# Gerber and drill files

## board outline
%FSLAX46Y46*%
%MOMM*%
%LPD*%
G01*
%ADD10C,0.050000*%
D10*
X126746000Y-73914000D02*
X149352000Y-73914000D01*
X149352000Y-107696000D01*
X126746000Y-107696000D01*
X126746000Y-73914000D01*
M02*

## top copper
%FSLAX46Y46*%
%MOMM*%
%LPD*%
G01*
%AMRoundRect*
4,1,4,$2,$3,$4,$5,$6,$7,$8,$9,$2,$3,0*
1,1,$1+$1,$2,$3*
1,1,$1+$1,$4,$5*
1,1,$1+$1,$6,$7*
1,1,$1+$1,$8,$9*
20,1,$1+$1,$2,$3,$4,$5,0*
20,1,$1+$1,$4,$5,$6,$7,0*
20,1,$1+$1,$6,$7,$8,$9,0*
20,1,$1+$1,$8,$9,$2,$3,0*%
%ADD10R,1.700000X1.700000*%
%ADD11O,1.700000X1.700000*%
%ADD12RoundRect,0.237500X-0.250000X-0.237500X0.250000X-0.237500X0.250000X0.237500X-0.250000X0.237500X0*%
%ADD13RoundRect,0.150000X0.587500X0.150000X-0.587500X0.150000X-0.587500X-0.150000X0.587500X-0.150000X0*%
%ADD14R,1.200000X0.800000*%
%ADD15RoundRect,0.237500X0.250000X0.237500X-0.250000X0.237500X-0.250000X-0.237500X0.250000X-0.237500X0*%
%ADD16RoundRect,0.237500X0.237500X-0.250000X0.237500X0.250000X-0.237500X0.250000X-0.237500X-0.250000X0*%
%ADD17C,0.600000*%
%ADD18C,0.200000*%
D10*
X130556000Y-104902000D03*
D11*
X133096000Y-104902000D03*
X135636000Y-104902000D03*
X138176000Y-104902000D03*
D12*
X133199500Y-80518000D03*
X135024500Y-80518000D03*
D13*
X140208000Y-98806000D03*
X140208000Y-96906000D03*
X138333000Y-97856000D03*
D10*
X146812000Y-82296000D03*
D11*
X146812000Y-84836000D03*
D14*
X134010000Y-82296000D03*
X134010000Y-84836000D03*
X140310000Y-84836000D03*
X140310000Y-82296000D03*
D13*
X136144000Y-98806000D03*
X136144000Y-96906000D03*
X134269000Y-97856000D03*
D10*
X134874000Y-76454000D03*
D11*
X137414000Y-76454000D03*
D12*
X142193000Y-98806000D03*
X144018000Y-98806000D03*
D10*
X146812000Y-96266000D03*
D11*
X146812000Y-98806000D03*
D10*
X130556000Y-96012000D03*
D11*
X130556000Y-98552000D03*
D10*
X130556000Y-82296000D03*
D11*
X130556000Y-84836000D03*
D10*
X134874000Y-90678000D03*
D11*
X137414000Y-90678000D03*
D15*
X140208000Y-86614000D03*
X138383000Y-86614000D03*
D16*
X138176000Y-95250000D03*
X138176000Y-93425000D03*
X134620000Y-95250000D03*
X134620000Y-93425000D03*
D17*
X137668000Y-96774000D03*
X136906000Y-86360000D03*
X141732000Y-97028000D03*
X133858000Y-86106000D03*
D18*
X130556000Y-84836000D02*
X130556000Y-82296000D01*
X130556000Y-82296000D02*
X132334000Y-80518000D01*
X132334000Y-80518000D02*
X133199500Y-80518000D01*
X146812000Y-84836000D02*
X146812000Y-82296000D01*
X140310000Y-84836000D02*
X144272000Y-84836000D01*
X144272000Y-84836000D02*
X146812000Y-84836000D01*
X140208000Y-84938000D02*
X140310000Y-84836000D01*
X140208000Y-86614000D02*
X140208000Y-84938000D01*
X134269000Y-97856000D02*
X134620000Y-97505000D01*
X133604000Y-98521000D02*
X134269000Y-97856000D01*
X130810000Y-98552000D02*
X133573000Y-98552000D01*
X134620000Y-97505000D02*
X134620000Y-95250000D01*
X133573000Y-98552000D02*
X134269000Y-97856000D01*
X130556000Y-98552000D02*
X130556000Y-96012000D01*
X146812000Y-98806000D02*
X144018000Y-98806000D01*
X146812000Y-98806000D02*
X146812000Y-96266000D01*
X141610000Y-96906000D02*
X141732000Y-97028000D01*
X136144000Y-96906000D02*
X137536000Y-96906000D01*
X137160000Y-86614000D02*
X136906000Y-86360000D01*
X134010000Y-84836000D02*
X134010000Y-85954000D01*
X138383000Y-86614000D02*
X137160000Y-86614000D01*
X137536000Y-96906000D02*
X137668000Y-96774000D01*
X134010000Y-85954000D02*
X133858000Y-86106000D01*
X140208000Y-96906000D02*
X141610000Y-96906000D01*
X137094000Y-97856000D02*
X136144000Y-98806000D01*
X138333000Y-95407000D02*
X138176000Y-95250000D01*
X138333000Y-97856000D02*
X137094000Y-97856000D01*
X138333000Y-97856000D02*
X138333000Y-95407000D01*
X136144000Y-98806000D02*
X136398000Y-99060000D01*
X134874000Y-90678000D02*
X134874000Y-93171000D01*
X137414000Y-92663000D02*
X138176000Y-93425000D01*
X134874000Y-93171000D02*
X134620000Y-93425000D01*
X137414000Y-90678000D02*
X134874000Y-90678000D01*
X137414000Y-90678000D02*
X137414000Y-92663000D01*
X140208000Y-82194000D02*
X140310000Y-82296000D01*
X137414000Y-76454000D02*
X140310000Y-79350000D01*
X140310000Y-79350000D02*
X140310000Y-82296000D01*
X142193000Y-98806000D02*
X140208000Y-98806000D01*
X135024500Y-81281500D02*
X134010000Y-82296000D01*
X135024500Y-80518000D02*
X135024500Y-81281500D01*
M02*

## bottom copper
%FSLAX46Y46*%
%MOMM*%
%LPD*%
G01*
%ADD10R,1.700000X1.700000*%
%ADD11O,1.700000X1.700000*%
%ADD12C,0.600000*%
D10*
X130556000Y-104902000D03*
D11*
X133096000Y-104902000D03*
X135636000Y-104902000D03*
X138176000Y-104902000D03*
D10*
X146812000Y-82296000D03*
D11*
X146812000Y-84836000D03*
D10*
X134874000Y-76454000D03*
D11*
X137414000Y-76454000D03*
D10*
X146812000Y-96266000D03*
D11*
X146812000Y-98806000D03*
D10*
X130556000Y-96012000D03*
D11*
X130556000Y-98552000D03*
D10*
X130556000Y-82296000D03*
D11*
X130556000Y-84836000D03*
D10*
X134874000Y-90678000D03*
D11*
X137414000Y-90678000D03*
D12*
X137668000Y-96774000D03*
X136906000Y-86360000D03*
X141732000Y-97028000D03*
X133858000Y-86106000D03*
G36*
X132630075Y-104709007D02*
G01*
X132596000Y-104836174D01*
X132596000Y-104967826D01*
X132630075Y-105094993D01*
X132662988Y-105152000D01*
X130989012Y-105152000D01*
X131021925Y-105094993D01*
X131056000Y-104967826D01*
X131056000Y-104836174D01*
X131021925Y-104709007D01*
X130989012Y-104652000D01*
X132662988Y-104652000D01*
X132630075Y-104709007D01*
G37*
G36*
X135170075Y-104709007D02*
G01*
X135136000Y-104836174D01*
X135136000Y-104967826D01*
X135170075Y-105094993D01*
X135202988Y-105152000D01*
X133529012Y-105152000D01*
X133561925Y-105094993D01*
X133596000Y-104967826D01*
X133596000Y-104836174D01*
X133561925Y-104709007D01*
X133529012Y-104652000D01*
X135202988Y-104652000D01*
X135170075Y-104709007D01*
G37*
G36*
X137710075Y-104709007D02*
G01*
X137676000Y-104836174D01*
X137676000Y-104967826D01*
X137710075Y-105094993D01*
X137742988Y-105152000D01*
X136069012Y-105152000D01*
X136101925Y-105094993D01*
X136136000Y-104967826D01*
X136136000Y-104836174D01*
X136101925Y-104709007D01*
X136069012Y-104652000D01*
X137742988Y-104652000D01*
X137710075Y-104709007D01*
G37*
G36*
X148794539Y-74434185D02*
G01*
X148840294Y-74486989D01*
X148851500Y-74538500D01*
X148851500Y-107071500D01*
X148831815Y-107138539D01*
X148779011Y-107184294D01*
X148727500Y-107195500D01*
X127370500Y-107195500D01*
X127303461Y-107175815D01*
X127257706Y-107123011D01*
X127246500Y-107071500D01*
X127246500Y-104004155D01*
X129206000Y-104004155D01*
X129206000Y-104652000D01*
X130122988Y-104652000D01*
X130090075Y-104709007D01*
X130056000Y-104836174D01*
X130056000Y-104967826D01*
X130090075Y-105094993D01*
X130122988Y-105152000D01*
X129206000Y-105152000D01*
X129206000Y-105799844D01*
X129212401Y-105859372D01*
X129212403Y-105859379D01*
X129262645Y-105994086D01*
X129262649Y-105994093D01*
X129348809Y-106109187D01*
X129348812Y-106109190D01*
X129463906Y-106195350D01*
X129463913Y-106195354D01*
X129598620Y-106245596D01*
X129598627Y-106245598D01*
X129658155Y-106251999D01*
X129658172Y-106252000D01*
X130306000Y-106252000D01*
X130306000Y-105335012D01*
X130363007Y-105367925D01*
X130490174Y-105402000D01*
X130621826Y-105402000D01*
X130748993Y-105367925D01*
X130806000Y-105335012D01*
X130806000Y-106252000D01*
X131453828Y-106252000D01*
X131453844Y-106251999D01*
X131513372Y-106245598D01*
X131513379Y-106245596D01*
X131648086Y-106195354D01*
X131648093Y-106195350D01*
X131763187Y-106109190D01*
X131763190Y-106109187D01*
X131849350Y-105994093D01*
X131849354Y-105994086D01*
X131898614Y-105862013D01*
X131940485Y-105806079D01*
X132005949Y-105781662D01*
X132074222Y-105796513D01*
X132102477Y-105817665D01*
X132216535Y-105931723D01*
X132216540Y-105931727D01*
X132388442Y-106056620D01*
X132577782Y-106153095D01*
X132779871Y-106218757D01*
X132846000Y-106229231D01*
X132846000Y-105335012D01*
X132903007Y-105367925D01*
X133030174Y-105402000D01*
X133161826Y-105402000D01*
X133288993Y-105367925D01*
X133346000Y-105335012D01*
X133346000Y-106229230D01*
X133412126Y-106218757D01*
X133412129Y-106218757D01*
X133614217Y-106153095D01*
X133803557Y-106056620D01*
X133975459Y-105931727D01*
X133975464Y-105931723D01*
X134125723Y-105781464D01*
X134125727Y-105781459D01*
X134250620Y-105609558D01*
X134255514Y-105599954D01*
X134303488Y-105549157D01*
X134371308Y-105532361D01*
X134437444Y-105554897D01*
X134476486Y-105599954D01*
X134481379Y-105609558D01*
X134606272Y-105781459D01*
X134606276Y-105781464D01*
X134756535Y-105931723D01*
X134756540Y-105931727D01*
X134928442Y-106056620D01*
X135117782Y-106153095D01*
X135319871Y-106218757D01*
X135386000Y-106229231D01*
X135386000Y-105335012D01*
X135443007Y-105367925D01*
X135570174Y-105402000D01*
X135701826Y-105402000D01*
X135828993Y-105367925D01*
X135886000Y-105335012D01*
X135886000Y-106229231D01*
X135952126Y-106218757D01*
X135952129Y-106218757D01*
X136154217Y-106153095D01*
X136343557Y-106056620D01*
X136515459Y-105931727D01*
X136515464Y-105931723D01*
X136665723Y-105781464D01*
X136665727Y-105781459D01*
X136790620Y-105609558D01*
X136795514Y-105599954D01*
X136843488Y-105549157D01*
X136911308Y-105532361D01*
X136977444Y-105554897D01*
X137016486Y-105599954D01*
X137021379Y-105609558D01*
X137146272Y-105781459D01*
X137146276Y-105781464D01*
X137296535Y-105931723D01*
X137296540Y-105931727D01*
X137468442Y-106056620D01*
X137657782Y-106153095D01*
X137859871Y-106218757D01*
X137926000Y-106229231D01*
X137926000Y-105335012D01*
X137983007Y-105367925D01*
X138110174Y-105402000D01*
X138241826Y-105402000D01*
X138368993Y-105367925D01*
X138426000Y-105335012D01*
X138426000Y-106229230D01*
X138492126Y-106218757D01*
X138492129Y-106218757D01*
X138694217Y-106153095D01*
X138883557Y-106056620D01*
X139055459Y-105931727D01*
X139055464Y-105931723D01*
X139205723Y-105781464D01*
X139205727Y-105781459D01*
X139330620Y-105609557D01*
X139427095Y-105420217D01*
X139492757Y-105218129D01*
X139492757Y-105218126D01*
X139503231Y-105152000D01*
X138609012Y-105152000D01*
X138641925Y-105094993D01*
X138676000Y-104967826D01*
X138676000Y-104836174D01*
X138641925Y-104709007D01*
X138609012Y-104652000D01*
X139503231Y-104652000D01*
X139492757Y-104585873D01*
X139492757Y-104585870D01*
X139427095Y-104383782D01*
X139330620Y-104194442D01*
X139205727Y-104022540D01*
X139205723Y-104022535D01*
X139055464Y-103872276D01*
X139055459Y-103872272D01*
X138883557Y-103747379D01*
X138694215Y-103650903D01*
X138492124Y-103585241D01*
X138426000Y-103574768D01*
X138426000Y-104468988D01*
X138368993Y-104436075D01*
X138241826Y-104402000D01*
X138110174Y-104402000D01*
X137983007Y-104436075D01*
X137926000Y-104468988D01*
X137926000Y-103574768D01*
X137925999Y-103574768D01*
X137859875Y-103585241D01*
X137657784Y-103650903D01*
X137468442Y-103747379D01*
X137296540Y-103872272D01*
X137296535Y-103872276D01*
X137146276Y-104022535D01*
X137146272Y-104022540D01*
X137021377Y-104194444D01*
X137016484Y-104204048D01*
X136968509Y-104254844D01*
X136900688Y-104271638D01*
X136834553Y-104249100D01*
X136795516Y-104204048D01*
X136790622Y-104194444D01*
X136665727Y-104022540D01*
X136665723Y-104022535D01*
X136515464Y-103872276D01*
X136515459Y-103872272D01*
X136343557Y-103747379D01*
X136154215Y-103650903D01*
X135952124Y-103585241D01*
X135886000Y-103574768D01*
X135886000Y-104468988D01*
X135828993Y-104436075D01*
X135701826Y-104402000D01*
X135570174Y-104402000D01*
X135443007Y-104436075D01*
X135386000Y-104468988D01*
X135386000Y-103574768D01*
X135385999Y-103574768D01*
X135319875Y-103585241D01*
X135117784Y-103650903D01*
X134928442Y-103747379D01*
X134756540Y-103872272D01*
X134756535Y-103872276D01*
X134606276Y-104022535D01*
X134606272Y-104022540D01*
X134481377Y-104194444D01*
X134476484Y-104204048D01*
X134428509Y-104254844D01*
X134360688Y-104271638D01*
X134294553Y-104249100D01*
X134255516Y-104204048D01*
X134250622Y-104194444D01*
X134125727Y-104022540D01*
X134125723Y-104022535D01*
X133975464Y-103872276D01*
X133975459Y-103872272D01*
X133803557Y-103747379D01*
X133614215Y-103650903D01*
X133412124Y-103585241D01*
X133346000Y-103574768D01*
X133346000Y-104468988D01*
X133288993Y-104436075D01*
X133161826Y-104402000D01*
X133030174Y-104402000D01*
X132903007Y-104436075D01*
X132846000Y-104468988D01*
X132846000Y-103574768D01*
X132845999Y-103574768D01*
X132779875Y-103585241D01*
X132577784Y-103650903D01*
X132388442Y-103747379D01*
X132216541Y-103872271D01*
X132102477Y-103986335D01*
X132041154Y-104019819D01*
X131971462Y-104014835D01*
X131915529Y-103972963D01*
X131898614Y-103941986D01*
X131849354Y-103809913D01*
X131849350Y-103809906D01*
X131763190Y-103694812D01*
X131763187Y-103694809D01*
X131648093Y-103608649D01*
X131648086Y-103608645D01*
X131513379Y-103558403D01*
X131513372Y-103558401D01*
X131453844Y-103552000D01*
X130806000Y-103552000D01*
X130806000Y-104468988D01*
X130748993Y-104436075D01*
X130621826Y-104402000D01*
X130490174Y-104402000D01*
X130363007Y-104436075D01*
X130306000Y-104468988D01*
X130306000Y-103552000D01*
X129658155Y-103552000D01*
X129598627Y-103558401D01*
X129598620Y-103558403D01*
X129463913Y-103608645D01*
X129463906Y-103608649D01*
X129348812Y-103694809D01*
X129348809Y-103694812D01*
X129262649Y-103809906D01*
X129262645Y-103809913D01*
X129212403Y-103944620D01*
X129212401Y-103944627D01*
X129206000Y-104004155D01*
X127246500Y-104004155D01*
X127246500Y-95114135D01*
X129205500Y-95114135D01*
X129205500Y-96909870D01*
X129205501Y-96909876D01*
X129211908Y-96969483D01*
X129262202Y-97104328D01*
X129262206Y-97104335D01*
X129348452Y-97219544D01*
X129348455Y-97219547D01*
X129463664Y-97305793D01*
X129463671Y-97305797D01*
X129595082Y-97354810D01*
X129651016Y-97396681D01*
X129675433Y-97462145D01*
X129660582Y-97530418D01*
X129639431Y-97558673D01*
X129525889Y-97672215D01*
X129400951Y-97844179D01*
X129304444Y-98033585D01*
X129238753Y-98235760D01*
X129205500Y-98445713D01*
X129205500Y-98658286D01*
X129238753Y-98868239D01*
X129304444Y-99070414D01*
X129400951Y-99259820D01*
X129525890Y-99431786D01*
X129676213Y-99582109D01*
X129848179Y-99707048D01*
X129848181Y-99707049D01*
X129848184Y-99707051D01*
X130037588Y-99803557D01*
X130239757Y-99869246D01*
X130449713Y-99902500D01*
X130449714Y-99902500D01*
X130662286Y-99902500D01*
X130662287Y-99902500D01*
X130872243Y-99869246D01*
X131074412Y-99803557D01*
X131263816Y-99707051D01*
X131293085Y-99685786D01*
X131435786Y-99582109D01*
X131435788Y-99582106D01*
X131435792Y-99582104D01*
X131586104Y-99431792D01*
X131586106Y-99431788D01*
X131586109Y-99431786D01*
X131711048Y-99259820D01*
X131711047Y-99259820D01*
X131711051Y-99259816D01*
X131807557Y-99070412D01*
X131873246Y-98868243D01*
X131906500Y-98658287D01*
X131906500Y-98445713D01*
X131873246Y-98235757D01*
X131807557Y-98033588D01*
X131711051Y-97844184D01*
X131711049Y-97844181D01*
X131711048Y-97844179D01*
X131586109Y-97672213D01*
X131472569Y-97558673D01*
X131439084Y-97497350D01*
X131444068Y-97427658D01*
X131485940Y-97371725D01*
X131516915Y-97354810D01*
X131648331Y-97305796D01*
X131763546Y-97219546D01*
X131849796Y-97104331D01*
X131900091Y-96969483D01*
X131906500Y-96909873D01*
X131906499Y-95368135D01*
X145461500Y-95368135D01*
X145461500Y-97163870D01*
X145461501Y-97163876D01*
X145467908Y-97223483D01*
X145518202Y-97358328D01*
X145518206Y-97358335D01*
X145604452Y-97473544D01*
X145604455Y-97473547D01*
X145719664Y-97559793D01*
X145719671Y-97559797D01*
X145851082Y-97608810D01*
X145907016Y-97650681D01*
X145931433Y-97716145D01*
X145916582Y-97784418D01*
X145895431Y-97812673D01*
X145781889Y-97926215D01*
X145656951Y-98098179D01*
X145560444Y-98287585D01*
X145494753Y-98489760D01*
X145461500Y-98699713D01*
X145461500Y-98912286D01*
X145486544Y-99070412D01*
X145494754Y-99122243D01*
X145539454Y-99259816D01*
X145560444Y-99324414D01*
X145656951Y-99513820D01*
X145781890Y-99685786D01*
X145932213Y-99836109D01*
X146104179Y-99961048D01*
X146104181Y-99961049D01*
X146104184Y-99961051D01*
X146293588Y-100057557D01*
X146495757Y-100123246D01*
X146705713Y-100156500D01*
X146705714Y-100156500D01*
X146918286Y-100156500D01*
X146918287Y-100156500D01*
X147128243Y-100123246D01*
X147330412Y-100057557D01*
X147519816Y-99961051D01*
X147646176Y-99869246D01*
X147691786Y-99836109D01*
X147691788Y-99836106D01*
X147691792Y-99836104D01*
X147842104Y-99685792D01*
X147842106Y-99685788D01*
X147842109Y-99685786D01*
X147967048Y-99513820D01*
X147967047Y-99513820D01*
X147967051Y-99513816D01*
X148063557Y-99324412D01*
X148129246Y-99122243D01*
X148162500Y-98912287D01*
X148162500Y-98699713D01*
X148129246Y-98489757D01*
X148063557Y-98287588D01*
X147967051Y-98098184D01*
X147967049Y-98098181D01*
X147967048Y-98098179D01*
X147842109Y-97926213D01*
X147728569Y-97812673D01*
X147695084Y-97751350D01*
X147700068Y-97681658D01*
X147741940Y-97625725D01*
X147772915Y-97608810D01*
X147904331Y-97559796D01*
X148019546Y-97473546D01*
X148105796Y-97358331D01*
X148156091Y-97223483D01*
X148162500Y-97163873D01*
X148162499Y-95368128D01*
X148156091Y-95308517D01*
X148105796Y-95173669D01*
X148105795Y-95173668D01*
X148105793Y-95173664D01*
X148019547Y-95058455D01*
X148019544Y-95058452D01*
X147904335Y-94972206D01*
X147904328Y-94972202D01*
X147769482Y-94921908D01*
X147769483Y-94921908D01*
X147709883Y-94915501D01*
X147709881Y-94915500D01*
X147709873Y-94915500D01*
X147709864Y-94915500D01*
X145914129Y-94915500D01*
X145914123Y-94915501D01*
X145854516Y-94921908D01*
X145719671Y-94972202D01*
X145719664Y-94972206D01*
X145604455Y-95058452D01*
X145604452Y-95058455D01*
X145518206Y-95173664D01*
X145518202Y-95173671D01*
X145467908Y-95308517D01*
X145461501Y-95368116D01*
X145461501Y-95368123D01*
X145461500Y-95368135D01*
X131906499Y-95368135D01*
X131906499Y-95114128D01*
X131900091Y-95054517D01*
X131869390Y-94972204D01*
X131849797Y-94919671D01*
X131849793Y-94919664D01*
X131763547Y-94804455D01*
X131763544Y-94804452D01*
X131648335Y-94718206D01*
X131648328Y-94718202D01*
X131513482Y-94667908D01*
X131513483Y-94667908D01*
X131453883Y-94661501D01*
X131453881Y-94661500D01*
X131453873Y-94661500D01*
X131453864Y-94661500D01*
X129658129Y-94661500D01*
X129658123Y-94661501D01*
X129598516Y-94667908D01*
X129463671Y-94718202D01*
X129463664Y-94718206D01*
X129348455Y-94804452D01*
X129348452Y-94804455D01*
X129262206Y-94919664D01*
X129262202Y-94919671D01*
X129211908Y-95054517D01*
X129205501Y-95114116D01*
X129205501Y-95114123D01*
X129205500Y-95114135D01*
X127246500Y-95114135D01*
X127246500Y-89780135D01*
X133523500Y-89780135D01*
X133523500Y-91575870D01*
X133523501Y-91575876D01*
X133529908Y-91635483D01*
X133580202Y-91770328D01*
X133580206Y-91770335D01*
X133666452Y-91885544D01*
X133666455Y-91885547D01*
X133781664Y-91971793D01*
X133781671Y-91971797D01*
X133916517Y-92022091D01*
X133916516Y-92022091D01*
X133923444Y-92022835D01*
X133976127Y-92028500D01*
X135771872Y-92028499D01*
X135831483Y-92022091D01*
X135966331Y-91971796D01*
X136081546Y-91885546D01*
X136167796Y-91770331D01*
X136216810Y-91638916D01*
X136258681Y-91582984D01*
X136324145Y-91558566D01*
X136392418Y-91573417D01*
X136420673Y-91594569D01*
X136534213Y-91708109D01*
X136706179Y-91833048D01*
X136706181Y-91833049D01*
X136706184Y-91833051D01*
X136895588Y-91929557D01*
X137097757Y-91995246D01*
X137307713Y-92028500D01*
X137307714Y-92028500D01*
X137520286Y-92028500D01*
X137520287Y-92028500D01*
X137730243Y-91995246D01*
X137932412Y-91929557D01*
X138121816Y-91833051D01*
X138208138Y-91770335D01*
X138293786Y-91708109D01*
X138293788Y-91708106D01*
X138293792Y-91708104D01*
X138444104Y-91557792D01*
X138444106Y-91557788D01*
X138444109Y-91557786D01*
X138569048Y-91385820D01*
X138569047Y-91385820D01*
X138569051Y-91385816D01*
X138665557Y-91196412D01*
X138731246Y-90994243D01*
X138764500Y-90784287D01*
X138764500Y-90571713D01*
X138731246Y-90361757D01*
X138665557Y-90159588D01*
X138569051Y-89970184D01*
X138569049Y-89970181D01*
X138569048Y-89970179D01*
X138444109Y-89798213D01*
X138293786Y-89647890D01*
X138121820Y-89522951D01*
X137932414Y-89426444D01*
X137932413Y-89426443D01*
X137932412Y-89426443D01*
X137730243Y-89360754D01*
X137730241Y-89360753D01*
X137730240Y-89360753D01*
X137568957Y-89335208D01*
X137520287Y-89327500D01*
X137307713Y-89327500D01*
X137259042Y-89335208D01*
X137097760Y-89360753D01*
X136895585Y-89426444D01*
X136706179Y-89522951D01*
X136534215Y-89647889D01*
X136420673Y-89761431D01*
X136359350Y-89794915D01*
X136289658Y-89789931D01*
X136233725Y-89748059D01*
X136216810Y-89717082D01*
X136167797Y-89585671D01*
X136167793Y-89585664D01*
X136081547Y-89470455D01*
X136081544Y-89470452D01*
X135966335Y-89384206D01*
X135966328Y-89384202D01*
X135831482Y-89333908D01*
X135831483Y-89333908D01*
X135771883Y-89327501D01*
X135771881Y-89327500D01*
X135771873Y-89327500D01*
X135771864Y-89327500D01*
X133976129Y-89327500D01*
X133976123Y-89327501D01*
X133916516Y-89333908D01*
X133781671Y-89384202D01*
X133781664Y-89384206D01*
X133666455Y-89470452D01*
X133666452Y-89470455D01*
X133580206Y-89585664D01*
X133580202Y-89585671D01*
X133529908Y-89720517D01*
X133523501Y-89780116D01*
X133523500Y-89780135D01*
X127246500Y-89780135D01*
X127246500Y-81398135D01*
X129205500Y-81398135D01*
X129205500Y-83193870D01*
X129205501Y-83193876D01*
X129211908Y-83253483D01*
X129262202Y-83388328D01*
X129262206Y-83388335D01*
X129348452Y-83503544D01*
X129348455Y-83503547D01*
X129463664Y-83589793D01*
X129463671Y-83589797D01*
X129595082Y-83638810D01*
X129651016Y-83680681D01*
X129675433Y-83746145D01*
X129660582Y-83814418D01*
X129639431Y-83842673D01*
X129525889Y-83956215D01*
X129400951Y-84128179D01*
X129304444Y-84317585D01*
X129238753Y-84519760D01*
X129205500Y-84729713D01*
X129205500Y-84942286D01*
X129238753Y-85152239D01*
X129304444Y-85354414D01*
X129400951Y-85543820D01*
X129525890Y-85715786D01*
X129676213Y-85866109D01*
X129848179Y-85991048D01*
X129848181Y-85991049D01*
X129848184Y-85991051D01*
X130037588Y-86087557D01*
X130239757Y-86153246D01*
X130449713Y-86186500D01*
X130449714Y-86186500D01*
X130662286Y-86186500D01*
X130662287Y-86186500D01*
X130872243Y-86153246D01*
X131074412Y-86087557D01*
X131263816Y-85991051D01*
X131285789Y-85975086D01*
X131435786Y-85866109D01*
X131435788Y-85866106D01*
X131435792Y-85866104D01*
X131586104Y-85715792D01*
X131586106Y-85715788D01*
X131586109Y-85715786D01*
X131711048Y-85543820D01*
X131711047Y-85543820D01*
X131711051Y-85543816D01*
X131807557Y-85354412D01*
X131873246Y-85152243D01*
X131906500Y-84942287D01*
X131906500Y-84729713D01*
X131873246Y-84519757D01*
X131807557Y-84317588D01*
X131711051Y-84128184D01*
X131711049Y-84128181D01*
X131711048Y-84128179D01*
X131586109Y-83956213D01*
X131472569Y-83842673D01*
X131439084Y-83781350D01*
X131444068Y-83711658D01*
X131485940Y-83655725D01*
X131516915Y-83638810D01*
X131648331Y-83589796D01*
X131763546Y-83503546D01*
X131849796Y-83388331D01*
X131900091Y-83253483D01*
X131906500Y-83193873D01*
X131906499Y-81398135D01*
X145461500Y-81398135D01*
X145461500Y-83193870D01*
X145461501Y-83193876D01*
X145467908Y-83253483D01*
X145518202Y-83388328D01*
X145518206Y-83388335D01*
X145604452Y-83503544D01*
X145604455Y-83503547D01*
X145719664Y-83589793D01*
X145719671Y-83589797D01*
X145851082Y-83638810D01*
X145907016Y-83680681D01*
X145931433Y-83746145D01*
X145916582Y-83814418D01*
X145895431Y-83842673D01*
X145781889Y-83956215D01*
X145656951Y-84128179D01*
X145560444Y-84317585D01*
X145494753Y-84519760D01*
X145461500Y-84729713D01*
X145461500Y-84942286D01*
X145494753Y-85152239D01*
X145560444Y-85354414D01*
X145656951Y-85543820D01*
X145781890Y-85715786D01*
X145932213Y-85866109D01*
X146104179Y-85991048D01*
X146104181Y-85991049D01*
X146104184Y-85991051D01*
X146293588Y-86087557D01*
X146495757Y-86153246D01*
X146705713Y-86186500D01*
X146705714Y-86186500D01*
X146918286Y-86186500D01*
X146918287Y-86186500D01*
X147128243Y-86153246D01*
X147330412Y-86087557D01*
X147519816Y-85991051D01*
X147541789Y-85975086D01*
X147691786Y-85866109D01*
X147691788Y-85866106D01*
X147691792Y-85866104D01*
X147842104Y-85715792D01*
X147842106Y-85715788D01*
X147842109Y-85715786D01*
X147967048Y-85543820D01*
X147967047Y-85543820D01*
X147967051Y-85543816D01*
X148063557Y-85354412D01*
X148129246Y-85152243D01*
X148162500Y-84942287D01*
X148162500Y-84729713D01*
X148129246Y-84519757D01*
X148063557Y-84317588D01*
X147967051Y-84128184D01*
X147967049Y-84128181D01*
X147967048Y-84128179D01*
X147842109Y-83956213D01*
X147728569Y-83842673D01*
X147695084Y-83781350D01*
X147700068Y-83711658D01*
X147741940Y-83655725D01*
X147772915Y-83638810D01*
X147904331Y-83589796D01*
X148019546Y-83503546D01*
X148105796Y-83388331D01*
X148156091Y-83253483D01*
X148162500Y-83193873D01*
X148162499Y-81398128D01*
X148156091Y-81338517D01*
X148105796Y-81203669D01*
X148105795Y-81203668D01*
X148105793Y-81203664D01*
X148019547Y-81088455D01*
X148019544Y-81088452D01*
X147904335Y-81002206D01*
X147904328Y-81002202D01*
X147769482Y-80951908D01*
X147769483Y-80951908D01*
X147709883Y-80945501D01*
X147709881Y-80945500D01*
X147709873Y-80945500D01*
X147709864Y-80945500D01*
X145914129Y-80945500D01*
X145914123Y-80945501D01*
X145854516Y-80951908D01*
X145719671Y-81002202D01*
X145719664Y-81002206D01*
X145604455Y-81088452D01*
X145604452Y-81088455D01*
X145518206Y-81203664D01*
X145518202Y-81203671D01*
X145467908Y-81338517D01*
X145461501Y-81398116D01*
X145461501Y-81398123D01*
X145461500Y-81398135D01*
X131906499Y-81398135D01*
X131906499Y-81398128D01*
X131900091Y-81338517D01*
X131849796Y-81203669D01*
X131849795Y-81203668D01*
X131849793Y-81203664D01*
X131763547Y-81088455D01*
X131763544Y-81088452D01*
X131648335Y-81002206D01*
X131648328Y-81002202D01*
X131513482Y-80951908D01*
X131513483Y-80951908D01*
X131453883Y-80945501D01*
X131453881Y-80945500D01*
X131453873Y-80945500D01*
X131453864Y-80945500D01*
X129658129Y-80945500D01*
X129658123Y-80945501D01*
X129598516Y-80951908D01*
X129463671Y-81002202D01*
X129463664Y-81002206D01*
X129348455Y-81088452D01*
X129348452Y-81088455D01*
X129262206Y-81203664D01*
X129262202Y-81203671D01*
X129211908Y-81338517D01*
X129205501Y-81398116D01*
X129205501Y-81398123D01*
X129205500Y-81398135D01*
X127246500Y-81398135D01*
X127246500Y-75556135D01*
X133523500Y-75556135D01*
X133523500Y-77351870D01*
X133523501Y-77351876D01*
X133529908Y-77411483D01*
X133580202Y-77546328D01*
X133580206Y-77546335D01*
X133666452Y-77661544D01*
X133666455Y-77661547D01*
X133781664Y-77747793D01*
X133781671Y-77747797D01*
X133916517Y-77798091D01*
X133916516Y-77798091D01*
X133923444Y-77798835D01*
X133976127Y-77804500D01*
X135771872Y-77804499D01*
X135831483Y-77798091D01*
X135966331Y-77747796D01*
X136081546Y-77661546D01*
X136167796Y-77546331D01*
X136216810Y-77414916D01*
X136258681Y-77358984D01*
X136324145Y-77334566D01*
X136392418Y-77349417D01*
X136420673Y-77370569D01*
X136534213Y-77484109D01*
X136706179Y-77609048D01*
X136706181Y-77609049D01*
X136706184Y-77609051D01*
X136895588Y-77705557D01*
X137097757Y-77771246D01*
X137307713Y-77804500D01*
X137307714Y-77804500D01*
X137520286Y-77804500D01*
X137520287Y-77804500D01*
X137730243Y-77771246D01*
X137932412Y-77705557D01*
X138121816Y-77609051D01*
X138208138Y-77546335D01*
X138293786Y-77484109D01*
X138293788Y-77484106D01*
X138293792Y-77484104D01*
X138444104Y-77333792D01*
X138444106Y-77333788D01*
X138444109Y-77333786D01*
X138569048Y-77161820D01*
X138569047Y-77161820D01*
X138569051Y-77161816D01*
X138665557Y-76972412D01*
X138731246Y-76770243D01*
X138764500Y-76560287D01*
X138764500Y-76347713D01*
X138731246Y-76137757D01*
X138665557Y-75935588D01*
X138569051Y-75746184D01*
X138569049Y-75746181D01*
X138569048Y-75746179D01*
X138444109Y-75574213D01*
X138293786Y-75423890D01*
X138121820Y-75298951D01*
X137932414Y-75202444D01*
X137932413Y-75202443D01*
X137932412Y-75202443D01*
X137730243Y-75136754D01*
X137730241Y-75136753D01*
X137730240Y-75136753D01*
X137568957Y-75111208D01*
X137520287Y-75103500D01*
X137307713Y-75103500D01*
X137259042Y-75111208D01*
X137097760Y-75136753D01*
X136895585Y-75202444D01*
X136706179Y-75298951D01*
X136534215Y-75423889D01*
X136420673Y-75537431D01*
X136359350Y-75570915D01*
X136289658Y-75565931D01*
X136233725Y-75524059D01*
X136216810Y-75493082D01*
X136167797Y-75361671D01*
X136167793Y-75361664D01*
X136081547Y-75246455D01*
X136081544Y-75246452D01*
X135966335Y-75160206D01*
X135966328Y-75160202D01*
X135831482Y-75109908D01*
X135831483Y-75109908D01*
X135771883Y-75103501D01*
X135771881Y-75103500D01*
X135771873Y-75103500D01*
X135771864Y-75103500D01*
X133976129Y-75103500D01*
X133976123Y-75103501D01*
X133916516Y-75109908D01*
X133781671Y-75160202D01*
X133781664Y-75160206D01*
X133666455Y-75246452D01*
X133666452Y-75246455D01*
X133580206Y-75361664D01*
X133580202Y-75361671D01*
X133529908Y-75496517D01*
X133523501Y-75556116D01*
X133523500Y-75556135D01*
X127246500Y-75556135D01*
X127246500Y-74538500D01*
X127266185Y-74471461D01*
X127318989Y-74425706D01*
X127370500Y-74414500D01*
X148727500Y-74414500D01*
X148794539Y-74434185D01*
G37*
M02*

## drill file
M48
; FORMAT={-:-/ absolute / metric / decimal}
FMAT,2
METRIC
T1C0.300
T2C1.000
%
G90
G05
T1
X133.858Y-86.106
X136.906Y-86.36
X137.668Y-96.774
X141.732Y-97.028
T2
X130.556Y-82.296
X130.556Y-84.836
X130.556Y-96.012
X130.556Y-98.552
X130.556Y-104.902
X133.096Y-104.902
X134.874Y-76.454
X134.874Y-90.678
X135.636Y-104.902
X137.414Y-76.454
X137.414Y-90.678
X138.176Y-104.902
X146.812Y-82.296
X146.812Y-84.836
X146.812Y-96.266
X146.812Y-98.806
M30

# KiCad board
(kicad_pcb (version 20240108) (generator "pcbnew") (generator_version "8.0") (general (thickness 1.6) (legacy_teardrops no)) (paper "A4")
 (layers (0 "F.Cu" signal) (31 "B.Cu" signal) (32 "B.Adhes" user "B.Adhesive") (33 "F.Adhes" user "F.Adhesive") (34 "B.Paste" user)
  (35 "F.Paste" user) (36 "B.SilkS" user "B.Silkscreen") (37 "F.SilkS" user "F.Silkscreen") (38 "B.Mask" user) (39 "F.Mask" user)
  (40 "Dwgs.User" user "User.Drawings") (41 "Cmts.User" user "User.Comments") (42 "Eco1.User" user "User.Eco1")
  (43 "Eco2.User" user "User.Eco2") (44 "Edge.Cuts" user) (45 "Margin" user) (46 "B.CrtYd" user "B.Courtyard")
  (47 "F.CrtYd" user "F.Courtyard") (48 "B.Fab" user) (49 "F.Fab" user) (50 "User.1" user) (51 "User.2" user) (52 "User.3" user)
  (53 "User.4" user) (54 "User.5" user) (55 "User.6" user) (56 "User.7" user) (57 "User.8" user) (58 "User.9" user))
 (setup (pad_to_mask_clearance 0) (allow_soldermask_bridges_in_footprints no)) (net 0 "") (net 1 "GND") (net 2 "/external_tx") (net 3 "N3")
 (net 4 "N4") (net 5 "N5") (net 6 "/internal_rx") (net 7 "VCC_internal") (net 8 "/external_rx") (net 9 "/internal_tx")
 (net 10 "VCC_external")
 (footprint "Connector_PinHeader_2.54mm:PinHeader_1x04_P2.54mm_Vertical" (layer "F.Cu") (at 130.556 104.902 90)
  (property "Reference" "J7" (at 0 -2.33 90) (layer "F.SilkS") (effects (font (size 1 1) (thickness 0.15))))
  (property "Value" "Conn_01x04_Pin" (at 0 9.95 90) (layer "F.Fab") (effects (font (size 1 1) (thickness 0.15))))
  (pad "1" thru_hole rect (at 0 0 90) (size 1.7 1.7) (drill 1) (layers "*.Cu" "*.Mask") (remove_unused_layers no) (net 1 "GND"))
  (pad "2" thru_hole oval (at 0 2.54 90) (size 1.7 1.7) (drill 1) (layers "*.Cu" "*.Mask") (remove_unused_layers no) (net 1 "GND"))
  (pad "3" thru_hole oval (at 0 5.08 90) (size 1.7 1.7) (drill 1) (layers "*.Cu" "*.Mask") (remove_unused_layers no) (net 1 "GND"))
  (pad "4" thru_hole oval (at 0 7.62 90) (size 1.7 1.7) (drill 1) (layers "*.Cu" "*.Mask") (remove_unused_layers no) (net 1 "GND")))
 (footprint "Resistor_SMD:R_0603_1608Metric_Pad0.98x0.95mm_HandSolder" (layer "F.Cu") (at 134.112 80.518)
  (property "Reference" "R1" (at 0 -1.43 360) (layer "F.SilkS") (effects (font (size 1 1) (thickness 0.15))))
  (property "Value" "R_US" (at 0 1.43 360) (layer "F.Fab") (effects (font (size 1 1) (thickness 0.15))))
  (pad "1" smd roundrect (at -0.9125 0) (size 0.975 0.95) (layers "F.Cu" "F.Paste" "F.Mask") (roundrect_rratio 0.25) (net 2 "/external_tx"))
  (pad "2" smd roundrect (at 0.9125 0) (size 0.975 0.95) (layers "F.Cu" "F.Paste" "F.Mask") (roundrect_rratio 0.25) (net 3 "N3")))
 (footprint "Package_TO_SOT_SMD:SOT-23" (layer "F.Cu") (at 139.2705 97.856 180)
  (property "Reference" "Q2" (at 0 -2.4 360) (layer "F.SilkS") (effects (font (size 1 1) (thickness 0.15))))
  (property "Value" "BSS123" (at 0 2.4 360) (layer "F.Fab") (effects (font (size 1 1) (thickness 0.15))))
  (pad "1" smd roundrect (at -0.9375 -0.95 180) (size 1.475 0.6) (layers "F.Cu" "F.Paste" "F.Mask") (roundrect_rratio 0.25) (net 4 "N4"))
  (pad "2" smd roundrect (at -0.9375 0.95 180) (size 1.475 0.6) (layers "F.Cu" "F.Paste" "F.Mask") (roundrect_rratio 0.25) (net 1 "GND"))
  (pad "3" smd roundrect (at 0.9375 0 180) (size 1.475 0.6) (layers "F.Cu" "F.Paste" "F.Mask") (roundrect_rratio 0.25) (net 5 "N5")))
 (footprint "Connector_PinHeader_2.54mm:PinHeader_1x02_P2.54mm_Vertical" (layer "F.Cu") (at 146.812 82.296)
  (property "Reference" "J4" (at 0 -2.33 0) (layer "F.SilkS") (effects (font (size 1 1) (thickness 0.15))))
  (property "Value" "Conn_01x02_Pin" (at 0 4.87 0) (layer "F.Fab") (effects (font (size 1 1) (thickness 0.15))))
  (pad "1" thru_hole rect (at 0 0) (size 1.7 1.7) (drill 1) (layers "*.Cu" "*.Mask") (remove_unused_layers no) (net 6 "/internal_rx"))
  (pad "2" thru_hole oval (at 0 2.54) (size 1.7 1.7) (drill 1) (layers "*.Cu" "*.Mask") (remove_unused_layers no) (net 6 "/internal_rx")))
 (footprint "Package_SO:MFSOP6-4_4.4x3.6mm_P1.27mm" (layer "F.Cu") (at 137.16 83.566)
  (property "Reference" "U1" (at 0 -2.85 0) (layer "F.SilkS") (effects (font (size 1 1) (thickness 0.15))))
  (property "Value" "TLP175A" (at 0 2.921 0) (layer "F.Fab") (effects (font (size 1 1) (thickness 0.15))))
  (pad "1" smd rect (at -3.15 -1.27) (size 1.2 0.8) (layers "F.Cu" "F.Paste" "F.Mask") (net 3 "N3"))
  (pad "3" smd rect (at -3.15 1.27) (size 1.2 0.8) (layers "F.Cu" "F.Paste" "F.Mask") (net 1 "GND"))
  (pad "4" smd rect (at 3.15 1.27) (size 1.2 0.8) (layers "F.Cu" "F.Paste" "F.Mask") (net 6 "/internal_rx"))
  (pad "6" smd rect (at 3.15 -1.27) (size 1.2 0.8) (layers "F.Cu" "F.Paste" "F.Mask") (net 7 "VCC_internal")))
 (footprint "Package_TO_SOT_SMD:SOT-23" (layer "F.Cu") (at 135.2065 97.856 180)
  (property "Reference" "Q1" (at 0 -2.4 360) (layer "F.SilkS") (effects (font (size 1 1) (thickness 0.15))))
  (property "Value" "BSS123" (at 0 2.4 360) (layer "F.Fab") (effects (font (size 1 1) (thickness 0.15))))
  (pad "1" smd roundrect (at -0.9375 -0.95 180) (size 1.475 0.6) (layers "F.Cu" "F.Paste" "F.Mask") (roundrect_rratio 0.25) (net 5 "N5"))
  (pad "2" smd roundrect (at -0.9375 0.95 180) (size 1.475 0.6) (layers "F.Cu" "F.Paste" "F.Mask") (roundrect_rratio 0.25) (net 1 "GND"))
  (pad "3" smd roundrect (at 0.9375 0 180) (size 1.475 0.6) (layers "F.Cu" "F.Paste" "F.Mask") (roundrect_rratio 0.25)
   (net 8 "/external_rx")))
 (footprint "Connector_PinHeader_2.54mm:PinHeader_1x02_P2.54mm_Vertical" (layer "F.Cu") (at 134.874 76.454 90)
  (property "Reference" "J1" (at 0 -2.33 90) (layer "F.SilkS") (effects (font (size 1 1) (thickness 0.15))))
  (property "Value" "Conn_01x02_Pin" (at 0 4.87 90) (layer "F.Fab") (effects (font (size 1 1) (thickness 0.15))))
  (pad "1" thru_hole rect (at 0 0 90) (size 1.7 1.7) (drill 1) (layers "*.Cu" "*.Mask") (remove_unused_layers no) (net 7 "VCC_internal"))
  (pad "2" thru_hole oval (at 0 2.54 90) (size 1.7 1.7) (drill 1) (layers "*.Cu" "*.Mask") (remove_unused_layers no) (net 7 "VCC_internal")))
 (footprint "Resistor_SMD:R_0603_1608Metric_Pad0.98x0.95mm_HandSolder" (layer "F.Cu") (at 143.1055 98.806)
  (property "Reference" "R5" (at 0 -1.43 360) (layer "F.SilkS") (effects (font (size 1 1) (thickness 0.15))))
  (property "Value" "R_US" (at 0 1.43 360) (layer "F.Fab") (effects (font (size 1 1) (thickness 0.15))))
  (pad "1" smd roundrect (at -0.9125 0) (size 0.975 0.95) (layers "F.Cu" "F.Paste" "F.Mask") (roundrect_rratio 0.25) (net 4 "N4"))
  (pad "2" smd roundrect (at 0.9125 0) (size 0.975 0.95) (layers "F.Cu" "F.Paste" "F.Mask") (roundrect_rratio 0.25) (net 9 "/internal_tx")))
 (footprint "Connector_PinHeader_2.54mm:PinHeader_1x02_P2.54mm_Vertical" (layer "F.Cu") (at 146.812 96.266)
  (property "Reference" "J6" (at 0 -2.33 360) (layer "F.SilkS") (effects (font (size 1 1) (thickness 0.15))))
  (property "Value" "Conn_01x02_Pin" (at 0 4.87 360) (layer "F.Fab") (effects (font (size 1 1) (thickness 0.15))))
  (pad "1" thru_hole rect (at 0 0) (size 1.7 1.7) (drill 1) (layers "*.Cu" "*.Mask") (remove_unused_layers no) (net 9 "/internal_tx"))
  (pad "2" thru_hole oval (at 0 2.54) (size 1.7 1.7) (drill 1) (layers "*.Cu" "*.Mask") (remove_unused_layers no) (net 9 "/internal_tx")))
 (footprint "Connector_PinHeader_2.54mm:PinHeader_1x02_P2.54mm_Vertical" (layer "F.Cu") (at 130.556 96.012)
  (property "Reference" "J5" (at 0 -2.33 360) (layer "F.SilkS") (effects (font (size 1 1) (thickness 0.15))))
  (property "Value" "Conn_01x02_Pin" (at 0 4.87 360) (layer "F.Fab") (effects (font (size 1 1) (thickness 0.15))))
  (pad "1" thru_hole rect (at 0 0) (size 1.7 1.7) (drill 1) (layers "*.Cu" "*.Mask") (remove_unused_layers no) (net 8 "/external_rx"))
  (pad "2" thru_hole oval (at 0 2.54) (size 1.7 1.7) (drill 1) (layers "*.Cu" "*.Mask") (remove_unused_layers no) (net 8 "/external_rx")))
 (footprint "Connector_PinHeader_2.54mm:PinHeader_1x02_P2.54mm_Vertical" (layer "F.Cu") (at 130.556 82.296)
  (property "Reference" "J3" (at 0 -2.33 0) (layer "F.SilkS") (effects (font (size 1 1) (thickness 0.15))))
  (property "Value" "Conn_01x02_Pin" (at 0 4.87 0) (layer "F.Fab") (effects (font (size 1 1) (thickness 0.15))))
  (pad "1" thru_hole rect (at 0 0) (size 1.7 1.7) (drill 1) (layers "*.Cu" "*.Mask") (remove_unused_layers no) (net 2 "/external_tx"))
  (pad "2" thru_hole oval (at 0 2.54) (size 1.7 1.7) (drill 1) (layers "*.Cu" "*.Mask") (remove_unused_layers no) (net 2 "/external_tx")))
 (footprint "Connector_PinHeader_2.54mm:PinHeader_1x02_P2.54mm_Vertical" (layer "F.Cu") (at 134.874 90.678 90)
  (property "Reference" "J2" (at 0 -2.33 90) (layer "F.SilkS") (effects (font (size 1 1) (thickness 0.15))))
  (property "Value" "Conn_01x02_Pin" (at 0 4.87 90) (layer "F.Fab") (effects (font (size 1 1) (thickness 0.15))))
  (pad "1" thru_hole rect (at 0 0 90) (size 1.7 1.7) (drill 1) (layers "*.Cu" "*.Mask") (remove_unused_layers no) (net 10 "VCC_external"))
  (pad "2" thru_hole oval (at 0 2.54 90) (size 1.7 1.7) (drill 1) (layers "*.Cu" "*.Mask") (remove_unused_layers no) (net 10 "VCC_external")))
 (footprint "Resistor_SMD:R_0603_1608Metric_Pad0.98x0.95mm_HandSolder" (layer "F.Cu") (at 139.2955 86.614 180)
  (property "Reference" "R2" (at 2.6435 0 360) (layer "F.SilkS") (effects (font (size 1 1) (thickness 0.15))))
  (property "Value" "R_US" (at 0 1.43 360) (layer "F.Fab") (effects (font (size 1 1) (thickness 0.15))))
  (pad "1" smd roundrect (at -0.9125 0 180) (size 0.975 0.95) (layers "F.Cu" "F.Paste" "F.Mask") (roundrect_rratio 0.25)
   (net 6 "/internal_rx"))
  (pad "2" smd roundrect (at 0.9125 0 180) (size 0.975 0.95) (layers "F.Cu" "F.Paste" "F.Mask") (roundrect_rratio 0.25) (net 1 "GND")))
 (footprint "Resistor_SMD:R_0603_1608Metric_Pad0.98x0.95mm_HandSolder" (layer "F.Cu") (at 138.176 94.3375 90)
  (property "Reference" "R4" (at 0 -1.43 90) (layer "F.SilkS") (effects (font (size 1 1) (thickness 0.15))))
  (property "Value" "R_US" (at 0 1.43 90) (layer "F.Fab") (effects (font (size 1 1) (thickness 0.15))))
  (pad "1" smd roundrect (at -0.9125 0 90) (size 0.975 0.95) (layers "F.Cu" "F.Paste" "F.Mask") (roundrect_rratio 0.25) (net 5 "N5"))
  (pad "2" smd roundrect (at 0.9125 0 90) (size 0.975 0.95) (layers "F.Cu" "F.Paste" "F.Mask") (roundrect_rratio 0.25)
   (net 10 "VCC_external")))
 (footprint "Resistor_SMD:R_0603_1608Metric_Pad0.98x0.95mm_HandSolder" (layer "F.Cu") (at 134.62 94.3375 90)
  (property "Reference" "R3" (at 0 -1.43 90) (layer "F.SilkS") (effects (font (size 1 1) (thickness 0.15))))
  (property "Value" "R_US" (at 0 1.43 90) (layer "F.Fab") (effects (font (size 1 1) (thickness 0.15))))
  (pad "1" smd roundrect (at -0.9125 0 90) (size 0.975 0.95) (layers "F.Cu" "F.Paste" "F.Mask") (roundrect_rratio 0.25)
   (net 8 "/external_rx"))
  (pad "2" smd roundrect (at 0.9125 0 90) (size 0.975 0.95) (layers "F.Cu" "F.Paste" "F.Mask") (roundrect_rratio 0.25)
   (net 10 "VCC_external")))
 (gr_rect (start 126.746 73.914) (end 149.352 107.696) (stroke (width 0.05) (type default)) (fill none) (layer "Edge.Cuts"))
 (segment (start 130.556 84.836) (end 130.556 82.296) (width 0.2) (layer "F.Cu") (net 2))
 (segment (start 130.556 82.296) (end 132.334 80.518) (width 0.2) (layer "F.Cu") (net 2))
 (segment (start 132.334 80.518) (end 133.1995 80.518) (width 0.2) (layer "F.Cu") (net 2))
 (segment (start 146.812 84.836) (end 146.812 82.296) (width 0.2) (layer "F.Cu") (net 6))
 (segment (start 140.31 84.836) (end 144.272 84.836) (width 0.2) (layer "F.Cu") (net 6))
 (segment (start 144.272 84.836) (end 146.812 84.836) (width 0.2) (layer "F.Cu") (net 6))
 (segment (start 140.208 84.938) (end 140.31 84.836) (width 0.2) (layer "F.Cu") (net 6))
 (segment (start 140.208 86.614) (end 140.208 84.938) (width 0.2) (layer "F.Cu") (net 6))
 (segment (start 134.269 97.856) (end 134.62 97.505) (width 0.2) (layer "F.Cu") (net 8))
 (segment (start 133.604 98.521) (end 134.269 97.856) (width 0.2) (layer "F.Cu") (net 8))
 (segment (start 130.81 98.552) (end 133.573 98.552) (width 0.2) (layer "F.Cu") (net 8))
 (segment (start 134.62 97.505) (end 134.62 95.25) (width 0.2) (layer "F.Cu") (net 8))
 (segment (start 133.573 98.552) (end 134.269 97.856) (width 0.2) (layer "F.Cu") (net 8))
 (segment (start 130.556 98.552) (end 130.556 96.012) (width 0.2) (layer "F.Cu") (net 8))
 (segment (start 146.812 98.806) (end 144.018 98.806) (width 0.2) (layer "F.Cu") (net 9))
 (segment (start 146.812 98.806) (end 146.812 96.266) (width 0.2) (layer "F.Cu") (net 9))
 (segment (start 141.61 96.906) (end 141.732 97.028) (width 0.2) (layer "F.Cu") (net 1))
 (segment (start 136.144 96.906) (end 137.536 96.906) (width 0.2) (layer "F.Cu") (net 1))
 (segment (start 137.16 86.614) (end 136.906 86.36) (width 0.2) (layer "F.Cu") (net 1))
 (segment (start 134.01 84.836) (end 134.01 85.954) (width 0.2) (layer "F.Cu") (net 1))
 (segment (start 138.383 86.614) (end 137.16 86.614) (width 0.2) (layer "F.Cu") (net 1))
 (segment (start 137.536 96.906) (end 137.668 96.774) (width 0.2) (layer "F.Cu") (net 1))
 (segment (start 134.01 85.954) (end 133.858 86.106) (width 0.2) (layer "F.Cu") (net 1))
 (segment (start 140.208 96.906) (end 141.61 96.906) (width 0.2) (layer "F.Cu") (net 1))
 (via (at 137.668 96.774) (size 0.6) (drill 0.3) (layers "F.Cu" "B.Cu") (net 1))
 (via (at 136.906 86.36) (size 0.6) (drill 0.3) (layers "F.Cu" "B.Cu") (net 1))
 (via (at 141.732 97.028) (size 0.6) (drill 0.3) (layers "F.Cu" "B.Cu") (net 1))
 (via (at 133.858 86.106) (size 0.6) (drill 0.3) (layers "F.Cu" "B.Cu") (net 1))
 (segment (start 137.094 97.856) (end 136.144 98.806) (width 0.2) (layer "F.Cu") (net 5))
 (segment (start 138.333 95.407) (end 138.176 95.25) (width 0.2) (layer "F.Cu") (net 5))
 (segment (start 138.333 97.856) (end 137.094 97.856) (width 0.2) (layer "F.Cu") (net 5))
 (segment (start 138.333 97.856) (end 138.333 95.407) (width 0.2) (layer "F.Cu") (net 5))
 (segment (start 136.144 98.806) (end 136.398 99.06) (width 0.2) (layer "F.Cu") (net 5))
 (segment (start 134.874 90.678) (end 134.874 93.171) (width 0.2) (layer "F.Cu") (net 10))
 (segment (start 137.414 92.663) (end 138.176 93.425) (width 0.2) (layer "F.Cu") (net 10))
 (segment (start 134.874 93.171) (end 134.62 93.425) (width 0.2) (layer "F.Cu") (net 10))
 (segment (start 137.414 90.678) (end 134.874 90.678) (width 0.2) (layer "F.Cu") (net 10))
 (segment (start 137.414 90.678) (end 137.414 92.663) (width 0.2) (layer "F.Cu") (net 10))
 (segment (start 140.208 82.194) (end 140.31 82.296) (width 0.2) (layer "F.Cu") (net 7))
 (segment (start 137.414 76.454) (end 140.31 79.35) (width 0.2) (layer "F.Cu") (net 7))
 (segment (start 140.31 79.35) (end 140.31 82.296) (width 0.2) (layer "F.Cu") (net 7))
 (segment (start 142.193 98.806) (end 140.208 98.806) (width 0.2) (layer "F.Cu") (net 4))
 (segment (start 135.0245 81.2815) (end 134.01 82.296) (width 0.2) (layer "F.Cu") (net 3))
 (segment (start 135.0245 80.518) (end 135.0245 81.2815) (width 0.2) (layer "F.Cu") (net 3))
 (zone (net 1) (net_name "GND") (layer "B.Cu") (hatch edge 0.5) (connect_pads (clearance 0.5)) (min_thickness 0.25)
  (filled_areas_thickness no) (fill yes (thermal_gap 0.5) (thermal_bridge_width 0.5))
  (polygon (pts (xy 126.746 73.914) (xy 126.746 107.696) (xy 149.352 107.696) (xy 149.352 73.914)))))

